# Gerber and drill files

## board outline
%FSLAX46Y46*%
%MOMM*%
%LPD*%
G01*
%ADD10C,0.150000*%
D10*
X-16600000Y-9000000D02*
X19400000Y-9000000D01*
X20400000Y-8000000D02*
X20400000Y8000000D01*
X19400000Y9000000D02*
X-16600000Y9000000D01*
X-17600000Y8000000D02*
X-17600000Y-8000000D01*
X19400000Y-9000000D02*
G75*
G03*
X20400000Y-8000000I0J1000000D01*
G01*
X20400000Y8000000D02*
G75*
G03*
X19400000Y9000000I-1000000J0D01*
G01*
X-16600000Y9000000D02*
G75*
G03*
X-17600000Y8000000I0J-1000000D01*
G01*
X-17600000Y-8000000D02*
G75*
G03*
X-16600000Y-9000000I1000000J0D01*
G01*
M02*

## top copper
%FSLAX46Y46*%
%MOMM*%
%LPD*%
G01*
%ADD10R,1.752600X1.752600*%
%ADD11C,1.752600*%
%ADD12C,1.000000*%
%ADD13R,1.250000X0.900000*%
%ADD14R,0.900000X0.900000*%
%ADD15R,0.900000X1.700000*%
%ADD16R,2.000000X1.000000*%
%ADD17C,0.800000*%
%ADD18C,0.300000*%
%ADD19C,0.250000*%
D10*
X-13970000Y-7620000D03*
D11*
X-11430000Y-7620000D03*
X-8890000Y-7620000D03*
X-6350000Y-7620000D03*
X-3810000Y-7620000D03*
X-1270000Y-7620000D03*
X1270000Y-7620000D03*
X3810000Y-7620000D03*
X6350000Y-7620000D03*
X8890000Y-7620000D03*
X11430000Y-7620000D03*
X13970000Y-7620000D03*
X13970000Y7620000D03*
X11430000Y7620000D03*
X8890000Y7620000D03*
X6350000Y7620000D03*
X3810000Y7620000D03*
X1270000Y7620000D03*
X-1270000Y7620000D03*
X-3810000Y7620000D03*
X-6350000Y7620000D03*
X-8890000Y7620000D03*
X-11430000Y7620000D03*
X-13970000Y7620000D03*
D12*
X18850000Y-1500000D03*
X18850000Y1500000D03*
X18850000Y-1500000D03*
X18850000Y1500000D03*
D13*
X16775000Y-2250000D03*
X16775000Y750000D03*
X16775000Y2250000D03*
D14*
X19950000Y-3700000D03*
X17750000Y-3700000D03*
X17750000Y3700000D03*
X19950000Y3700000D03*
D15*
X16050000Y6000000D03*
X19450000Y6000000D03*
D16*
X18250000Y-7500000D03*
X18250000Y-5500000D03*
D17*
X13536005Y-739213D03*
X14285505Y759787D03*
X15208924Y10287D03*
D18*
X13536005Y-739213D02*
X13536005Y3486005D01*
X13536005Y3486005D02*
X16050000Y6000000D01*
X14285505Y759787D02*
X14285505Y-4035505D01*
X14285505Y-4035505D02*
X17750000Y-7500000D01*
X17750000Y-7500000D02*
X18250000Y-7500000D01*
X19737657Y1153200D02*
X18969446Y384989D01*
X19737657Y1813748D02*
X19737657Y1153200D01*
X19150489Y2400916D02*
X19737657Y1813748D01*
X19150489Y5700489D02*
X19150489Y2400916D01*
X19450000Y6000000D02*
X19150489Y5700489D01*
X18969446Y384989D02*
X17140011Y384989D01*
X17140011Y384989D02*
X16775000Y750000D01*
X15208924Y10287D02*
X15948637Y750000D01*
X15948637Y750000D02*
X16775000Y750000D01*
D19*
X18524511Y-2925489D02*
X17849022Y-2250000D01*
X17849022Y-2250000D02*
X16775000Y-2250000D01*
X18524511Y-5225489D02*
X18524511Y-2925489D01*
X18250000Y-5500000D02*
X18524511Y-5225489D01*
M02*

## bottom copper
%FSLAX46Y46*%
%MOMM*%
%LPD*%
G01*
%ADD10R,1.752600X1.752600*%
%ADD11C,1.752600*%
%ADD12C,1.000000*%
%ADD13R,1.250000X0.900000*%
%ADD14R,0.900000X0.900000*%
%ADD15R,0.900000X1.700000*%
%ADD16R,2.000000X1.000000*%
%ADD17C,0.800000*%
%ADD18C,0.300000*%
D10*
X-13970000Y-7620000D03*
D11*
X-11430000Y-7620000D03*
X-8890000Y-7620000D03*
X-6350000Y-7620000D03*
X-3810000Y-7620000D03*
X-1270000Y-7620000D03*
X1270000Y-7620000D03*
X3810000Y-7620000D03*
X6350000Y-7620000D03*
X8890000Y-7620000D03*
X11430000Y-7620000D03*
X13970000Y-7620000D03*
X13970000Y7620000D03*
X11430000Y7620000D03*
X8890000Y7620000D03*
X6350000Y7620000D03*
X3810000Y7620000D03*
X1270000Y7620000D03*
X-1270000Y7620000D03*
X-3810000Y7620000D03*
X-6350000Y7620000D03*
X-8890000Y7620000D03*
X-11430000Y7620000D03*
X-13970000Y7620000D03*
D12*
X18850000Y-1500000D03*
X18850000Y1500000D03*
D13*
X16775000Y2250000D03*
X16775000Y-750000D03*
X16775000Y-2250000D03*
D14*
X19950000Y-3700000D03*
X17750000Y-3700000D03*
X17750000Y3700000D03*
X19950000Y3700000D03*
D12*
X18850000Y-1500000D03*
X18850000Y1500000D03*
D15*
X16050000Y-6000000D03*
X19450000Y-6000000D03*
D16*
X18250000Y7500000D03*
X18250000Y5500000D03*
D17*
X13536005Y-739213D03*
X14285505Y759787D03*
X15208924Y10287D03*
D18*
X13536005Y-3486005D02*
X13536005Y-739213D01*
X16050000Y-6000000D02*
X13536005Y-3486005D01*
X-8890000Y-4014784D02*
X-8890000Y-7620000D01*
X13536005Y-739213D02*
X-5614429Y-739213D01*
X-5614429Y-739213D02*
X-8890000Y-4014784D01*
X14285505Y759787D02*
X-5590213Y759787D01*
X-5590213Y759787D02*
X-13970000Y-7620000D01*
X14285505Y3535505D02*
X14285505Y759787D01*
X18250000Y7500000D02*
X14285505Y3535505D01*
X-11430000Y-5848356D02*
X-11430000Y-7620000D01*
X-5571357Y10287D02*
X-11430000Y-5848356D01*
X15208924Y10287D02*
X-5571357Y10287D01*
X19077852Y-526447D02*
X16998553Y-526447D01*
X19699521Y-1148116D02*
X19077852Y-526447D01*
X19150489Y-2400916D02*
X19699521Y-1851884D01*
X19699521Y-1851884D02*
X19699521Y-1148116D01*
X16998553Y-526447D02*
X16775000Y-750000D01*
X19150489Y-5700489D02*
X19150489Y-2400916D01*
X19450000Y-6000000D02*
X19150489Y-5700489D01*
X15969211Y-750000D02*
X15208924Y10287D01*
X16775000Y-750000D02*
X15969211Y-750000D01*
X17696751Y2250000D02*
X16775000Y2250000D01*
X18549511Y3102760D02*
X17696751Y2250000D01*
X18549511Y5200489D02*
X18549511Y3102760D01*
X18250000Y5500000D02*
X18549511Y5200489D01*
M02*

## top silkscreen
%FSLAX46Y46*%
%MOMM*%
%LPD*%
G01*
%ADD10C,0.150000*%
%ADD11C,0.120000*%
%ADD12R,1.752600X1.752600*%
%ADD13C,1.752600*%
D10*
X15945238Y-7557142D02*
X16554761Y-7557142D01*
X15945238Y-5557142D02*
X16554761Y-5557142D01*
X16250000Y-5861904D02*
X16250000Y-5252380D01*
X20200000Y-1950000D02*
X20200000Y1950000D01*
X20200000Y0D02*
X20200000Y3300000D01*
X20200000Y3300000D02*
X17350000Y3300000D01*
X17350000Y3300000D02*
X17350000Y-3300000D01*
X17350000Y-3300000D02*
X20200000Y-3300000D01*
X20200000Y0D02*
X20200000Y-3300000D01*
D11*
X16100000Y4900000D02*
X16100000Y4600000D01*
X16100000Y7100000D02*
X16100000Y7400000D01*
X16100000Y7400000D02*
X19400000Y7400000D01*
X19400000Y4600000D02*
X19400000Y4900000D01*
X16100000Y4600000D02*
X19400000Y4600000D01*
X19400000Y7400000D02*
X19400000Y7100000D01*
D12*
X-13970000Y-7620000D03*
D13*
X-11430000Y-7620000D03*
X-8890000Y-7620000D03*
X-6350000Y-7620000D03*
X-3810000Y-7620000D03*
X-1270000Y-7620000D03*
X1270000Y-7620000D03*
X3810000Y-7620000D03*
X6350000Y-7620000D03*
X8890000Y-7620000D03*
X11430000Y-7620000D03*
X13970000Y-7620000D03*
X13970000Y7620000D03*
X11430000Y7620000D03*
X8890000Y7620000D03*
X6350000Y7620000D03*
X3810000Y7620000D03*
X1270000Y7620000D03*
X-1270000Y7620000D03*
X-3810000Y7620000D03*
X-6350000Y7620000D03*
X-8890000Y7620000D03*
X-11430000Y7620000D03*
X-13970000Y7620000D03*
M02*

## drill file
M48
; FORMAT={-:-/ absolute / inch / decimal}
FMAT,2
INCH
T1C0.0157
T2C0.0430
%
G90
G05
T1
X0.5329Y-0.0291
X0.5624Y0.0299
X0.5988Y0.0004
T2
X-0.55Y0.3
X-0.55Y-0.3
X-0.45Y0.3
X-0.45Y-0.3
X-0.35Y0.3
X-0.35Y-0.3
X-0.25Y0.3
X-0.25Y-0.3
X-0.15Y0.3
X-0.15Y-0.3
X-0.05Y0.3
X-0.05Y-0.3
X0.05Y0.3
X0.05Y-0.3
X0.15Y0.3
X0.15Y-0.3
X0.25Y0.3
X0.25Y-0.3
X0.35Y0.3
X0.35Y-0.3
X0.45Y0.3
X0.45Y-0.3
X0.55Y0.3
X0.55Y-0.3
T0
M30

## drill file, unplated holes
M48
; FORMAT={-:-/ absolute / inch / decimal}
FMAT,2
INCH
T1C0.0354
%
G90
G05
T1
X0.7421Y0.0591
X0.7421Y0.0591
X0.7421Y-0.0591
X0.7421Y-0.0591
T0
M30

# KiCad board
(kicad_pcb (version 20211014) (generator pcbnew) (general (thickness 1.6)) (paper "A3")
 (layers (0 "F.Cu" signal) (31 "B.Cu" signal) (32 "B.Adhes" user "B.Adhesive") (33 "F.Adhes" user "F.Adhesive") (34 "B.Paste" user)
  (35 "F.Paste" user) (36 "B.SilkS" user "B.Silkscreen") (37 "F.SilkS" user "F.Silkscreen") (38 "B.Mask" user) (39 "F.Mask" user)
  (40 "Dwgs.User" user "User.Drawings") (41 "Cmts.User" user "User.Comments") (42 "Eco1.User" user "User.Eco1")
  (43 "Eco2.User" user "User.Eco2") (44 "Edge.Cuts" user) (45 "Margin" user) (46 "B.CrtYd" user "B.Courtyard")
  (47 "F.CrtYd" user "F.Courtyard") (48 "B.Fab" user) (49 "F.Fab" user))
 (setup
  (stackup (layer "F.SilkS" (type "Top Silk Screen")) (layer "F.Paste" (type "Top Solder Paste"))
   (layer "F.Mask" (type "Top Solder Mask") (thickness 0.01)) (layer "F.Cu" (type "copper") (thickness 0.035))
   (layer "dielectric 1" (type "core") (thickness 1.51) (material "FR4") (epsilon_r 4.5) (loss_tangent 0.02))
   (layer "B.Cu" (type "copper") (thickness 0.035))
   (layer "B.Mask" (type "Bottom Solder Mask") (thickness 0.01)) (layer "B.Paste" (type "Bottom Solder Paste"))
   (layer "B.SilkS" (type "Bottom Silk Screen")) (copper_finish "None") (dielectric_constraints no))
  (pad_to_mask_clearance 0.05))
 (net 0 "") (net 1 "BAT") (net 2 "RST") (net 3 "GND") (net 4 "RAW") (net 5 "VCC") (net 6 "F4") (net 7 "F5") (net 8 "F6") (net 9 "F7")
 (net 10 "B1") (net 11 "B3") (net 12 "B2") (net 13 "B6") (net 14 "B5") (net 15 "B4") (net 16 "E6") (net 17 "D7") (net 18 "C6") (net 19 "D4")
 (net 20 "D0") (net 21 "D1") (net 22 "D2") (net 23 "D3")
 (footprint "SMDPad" (layer "F.Cu") (at 18.25 -5.5)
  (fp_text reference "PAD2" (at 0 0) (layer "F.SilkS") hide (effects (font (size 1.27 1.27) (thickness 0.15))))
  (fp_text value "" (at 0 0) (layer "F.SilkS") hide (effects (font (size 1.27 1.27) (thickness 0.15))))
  (pad "1" smd rect locked (at 0 0) (size 2 1) (layers "B.Cu" "B.Paste" "B.Mask") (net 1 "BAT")))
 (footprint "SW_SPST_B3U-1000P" (layer "F.Cu") (at 17.75 -6)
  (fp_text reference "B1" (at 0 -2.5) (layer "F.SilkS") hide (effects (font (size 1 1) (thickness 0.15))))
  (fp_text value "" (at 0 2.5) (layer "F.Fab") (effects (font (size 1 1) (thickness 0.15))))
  (fp_line (start 1.65 -1.4) (end 1.65 -1.1) (layer "F.SilkS") (width 0.12))
  (fp_line (start -1.65 1.1) (end -1.65 1.4) (layer "F.SilkS") (width 0.12))
  (fp_line (start -1.65 1.4) (end 1.65 1.4) (layer "F.SilkS") (width 0.12))
  (fp_line (start 1.65 1.4) (end 1.65 1.1) (layer "F.SilkS") (width 0.12))
  (fp_line (start -1.65 -1.4) (end 1.65 -1.4) (layer "F.SilkS") (width 0.12))
  (fp_line (start -1.65 -1.1) (end -1.65 -1.4) (layer "F.SilkS") (width 0.12))
  (pad "1" smd rect locked (at -1.7 0) (size 0.9 1.7) (layers "F.Cu" "F.Paste" "F.Mask") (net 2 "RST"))
  (pad "2" smd rect locked (at 1.7 0) (size 0.9 1.7) (layers "F.Cu" "F.Paste" "F.Mask") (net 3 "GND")))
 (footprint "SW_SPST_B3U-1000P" (layer "F.Cu") (at 17.75 6)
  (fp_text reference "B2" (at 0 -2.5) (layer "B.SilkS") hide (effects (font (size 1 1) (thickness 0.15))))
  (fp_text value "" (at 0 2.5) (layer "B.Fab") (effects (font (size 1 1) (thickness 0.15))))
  (pad "1" smd rect locked (at -1.7 0) (size 0.9 1.7) (layers "B.Cu" "B.Paste" "B.Mask") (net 2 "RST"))
  (pad "2" smd rect locked (at 1.7 0) (size 0.9 1.7) (layers "B.Cu" "B.Paste" "B.Mask") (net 3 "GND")))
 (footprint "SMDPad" (layer "F.Cu") (at 18.25 5.5)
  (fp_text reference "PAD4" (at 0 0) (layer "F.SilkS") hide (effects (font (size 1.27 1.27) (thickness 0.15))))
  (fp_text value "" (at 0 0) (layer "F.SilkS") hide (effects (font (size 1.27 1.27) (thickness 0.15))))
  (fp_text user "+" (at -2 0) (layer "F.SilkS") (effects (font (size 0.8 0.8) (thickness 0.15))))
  (pad "1" smd rect locked (at 0 0) (size 2 1) (layers "F.Cu" "F.Paste" "F.Mask") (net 1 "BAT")))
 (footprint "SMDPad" (layer "F.Cu") (at 18.25 -7.5)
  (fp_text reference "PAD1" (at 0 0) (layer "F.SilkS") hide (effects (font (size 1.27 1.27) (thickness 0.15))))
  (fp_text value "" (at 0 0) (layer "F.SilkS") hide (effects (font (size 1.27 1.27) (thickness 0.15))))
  (pad "1" smd rect locked (at 0 0) (size 2 1) (layers "B.Cu" "B.Paste" "B.Mask") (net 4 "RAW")))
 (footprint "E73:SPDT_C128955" (layer "F.Cu") (at 18.85 0 -90)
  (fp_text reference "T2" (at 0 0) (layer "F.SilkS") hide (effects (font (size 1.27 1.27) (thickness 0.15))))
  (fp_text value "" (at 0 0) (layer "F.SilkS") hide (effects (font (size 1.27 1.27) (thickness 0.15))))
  (fp_line (start 0 -1.35) (end -3.3 -1.35) (layer "F.SilkS") (width 0.15))
  (fp_line (start 3.3 1.5) (end 3.3 -1.35) (layer "F.SilkS") (width 0.15))
  (fp_line (start -3.3 -1.35) (end -3.3 1.5) (layer "F.SilkS") (width 0.15))
  (fp_line (start -3.3 1.5) (end 3.3 1.5) (layer "F.SilkS") (width 0.15))
  (fp_line (start 0 -1.35) (end 3.3 -1.35) (layer "F.SilkS") (width 0.15))
  (fp_line (start 1.95 -1.35) (end -1.95 -1.35) (layer "F.SilkS") (width 0.15))
  (pad "" np_thru_hole circle locked (at 1.5 0) (size 1 1) (drill 0.9) (layers *.Cu *.Mask))
  (pad "" smd rect locked (at 3.7 -1.1 270) (size 0.9 0.9) (layers "F.Cu" "F.Paste" "F.Mask"))
  (pad "" smd rect locked (at 3.7 1.1 270) (size 0.9 0.9) (layers "F.Cu" "F.Paste" "F.Mask"))
  (pad "" np_thru_hole circle locked (at -1.5 0) (size 1 1) (drill 0.9) (layers *.Cu *.Mask))
  (pad "" smd rect locked (at -3.7 1.1 270) (size 0.9 0.9) (layers "F.Cu" "F.Paste" "F.Mask"))
  (pad "" smd rect locked (at -3.7 -1.1 270) (size 0.9 0.9) (layers "F.Cu" "F.Paste" "F.Mask"))
  (pad "1" smd rect locked (at 2.25 2.075 270) (size 0.9 1.25) (layers "F.Cu" "F.Paste" "F.Mask") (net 1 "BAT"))
  (pad "2" smd rect locked (at -0.75 2.075 270) (size 0.9 1.25) (layers "F.Cu" "F.Paste" "F.Mask") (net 3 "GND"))
  (pad "3" smd rect locked (at -2.25 2.075 270) (size 0.9 1.25) (layers "F.Cu" "F.Paste" "F.Mask")))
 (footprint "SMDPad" (layer "F.Cu") (at 18.25 7.5)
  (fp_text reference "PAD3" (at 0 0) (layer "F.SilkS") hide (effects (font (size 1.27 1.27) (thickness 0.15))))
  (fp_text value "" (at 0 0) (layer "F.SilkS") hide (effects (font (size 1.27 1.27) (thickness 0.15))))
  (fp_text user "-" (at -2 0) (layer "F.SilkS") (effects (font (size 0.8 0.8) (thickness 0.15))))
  (pad "1" smd rect locked (at 0 0) (size 2 1) (layers "F.Cu" "F.Paste" "F.Mask") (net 4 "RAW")))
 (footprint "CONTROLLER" (layer "F.Cu") (at 0 0)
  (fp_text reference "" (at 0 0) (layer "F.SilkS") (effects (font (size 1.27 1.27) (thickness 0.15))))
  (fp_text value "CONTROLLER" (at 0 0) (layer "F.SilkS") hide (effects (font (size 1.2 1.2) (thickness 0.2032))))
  (pad "1" thru_hole rect locked (at -13.97 7.62) (size 1.7526 1.7526) (drill 1.0922) (layers *.Cu *.SilkS *.Mask) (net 4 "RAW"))
  (pad "2" thru_hole circle locked (at -11.43 7.62) (size 1.7526 1.7526) (drill 1.0922) (layers *.Cu *.SilkS *.Mask) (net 3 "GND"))
  (pad "3" thru_hole circle locked (at -8.89 7.62) (size 1.7526 1.7526) (drill 1.0922) (layers *.Cu *.SilkS *.Mask) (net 2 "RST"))
  (pad "4" thru_hole circle locked (at -6.35 7.62) (size 1.7526 1.7526) (drill 1.0922) (layers *.Cu *.SilkS *.Mask) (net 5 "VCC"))
  (pad "5" thru_hole circle locked (at -3.81 7.62) (size 1.7526 1.7526) (drill 1.0922) (layers *.Cu *.SilkS *.Mask) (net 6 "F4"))
  (pad "6" thru_hole circle locked (at -1.27 7.62) (size 1.7526 1.7526) (drill 1.0922) (layers *.Cu *.SilkS *.Mask) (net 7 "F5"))
  (pad "7" thru_hole circle locked (at 1.27 7.62) (size 1.7526 1.7526) (drill 1.0922) (layers *.Cu *.SilkS *.Mask) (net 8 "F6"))
  (pad "8" thru_hole circle locked (at 3.81 7.62) (size 1.7526 1.7526) (drill 1.0922) (layers *.Cu *.SilkS *.Mask) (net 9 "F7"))
  (pad "9" thru_hole circle locked (at 6.35 7.62) (size 1.7526 1.7526) (drill 1.0922) (layers *.Cu *.SilkS *.Mask) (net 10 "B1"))
  (pad "10" thru_hole circle locked (at 8.89 7.62) (size 1.7526 1.7526) (drill 1.0922) (layers *.Cu *.SilkS *.Mask) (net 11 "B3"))
  (pad "11" thru_hole circle locked (at 11.43 7.62) (size 1.7526 1.7526) (drill 1.0922) (layers *.Cu *.SilkS *.Mask) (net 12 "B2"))
  (pad "12" thru_hole circle locked (at 13.97 7.62) (size 1.7526 1.7526) (drill 1.0922) (layers *.Cu *.SilkS *.Mask) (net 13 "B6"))
  (pad "13" thru_hole circle locked (at 13.97 -7.62) (size 1.7526 1.7526) (drill 1.0922) (layers *.Cu *.SilkS *.Mask) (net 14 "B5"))
  (pad "14" thru_hole circle locked (at 11.43 -7.62) (size 1.7526 1.7526) (drill 1.0922) (layers *.Cu *.SilkS *.Mask) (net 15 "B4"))
  (pad "15" thru_hole circle locked (at 8.89 -7.62) (size 1.7526 1.7526) (drill 1.0922) (layers *.Cu *.SilkS *.Mask) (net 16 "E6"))
  (pad "16" thru_hole circle locked (at 6.35 -7.62) (size 1.7526 1.7526) (drill 1.0922) (layers *.Cu *.SilkS *.Mask) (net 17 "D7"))
  (pad "17" thru_hole circle locked (at 3.81 -7.62) (size 1.7526 1.7526) (drill 1.0922) (layers *.Cu *.SilkS *.Mask) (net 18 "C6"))
  (pad "18" thru_hole circle locked (at 1.27 -7.62) (size 1.7526 1.7526) (drill 1.0922) (layers *.Cu *.SilkS *.Mask) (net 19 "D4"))
  (pad "19" thru_hole circle locked (at -1.27 -7.62) (size 1.7526 1.7526) (drill 1.0922) (layers *.Cu *.SilkS *.Mask) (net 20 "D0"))
  (pad "20" thru_hole circle locked (at -3.81 -7.62) (size 1.7526 1.7526) (drill 1.0922) (layers *.Cu *.SilkS *.Mask) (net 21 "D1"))
  (pad "21" thru_hole circle locked (at -6.35 -7.62) (size 1.7526 1.7526) (drill 1.0922) (layers *.Cu *.SilkS *.Mask) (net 3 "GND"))
  (pad "22" thru_hole circle locked (at -8.89 -7.62) (size 1.7526 1.7526) (drill 1.0922) (layers *.Cu *.SilkS *.Mask) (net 3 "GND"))
  (pad "23" thru_hole circle locked (at -11.43 -7.62) (size 1.7526 1.7526) (drill 1.0922) (layers *.Cu *.SilkS *.Mask) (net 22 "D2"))
  (pad "24" thru_hole circle locked (at -13.97 -7.62) (size 1.7526 1.7526) (drill 1.0922) (layers *.Cu *.SilkS *.Mask) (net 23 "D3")))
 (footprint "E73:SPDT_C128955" (layer "B.Cu") (at 18.85 0 -90)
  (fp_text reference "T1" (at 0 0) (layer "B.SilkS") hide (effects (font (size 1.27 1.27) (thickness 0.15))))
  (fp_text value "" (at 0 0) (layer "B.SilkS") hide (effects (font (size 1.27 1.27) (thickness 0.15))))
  (pad "" smd rect locked (at 3.7 -1.1 270) (size 0.9 0.9) (layers "B.Cu" "B.Paste" "B.Mask"))
  (pad "" smd rect locked (at -3.7 -1.1 270) (size 0.9 0.9) (layers "B.Cu" "B.Paste" "B.Mask"))
  (pad "" np_thru_hole circle locked (at 1.5 0) (size 1 1) (drill 0.9) (layers *.Cu *.Mask))
  (pad "" np_thru_hole circle locked (at -1.5 0) (size 1 1) (drill 0.9) (layers *.Cu *.Mask))
  (pad "" smd rect locked (at 3.7 1.1 270) (size 0.9 0.9) (layers "B.Cu" "B.Paste" "B.Mask"))
  (pad "" smd rect locked (at -3.7 1.1 270) (size 0.9 0.9) (layers "B.Cu" "B.Paste" "B.Mask"))
  (pad "1" smd rect locked (at -2.25 2.075 270) (size 0.9 1.25) (layers "B.Cu" "B.Paste" "B.Mask") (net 1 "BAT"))
  (pad "2" smd rect locked (at 0.75 2.075 270) (size 0.9 1.25) (layers "B.Cu" "B.Paste" "B.Mask") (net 3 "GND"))
  (pad "3" smd rect locked (at 2.25 2.075 270) (size 0.9 1.25) (layers "B.Cu" "B.Paste" "B.Mask")))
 (gr_line (start -17.6 -8) (end -17.6 8) (layer "Edge.Cuts") (width 0.15))
 (gr_arc (start -16.6 9) (mid -17.307107 8.707107) (end -17.6 8) (layer "Edge.Cuts") (width 0.15))
 (gr_arc (start 20.4 8) (mid 20.107107 8.707107) (end 19.4 9) (layer "Edge.Cuts") (width 0.15))
 (gr_line (start 19.4 -9) (end -16.6 -9) (layer "Edge.Cuts") (width 0.15))
 (gr_line (start 20.4 8) (end 20.4 -8) (layer "Edge.Cuts") (width 0.15))
 (gr_line (start -16.6 9) (end 19.4 9) (layer "Edge.Cuts") (width 0.15))
 (gr_arc (start -17.6 -8) (mid -17.307107 -8.707107) (end -16.6 -9) (layer "Edge.Cuts") (width 0.15))
 (gr_arc (start 19.4 -9) (mid 20.107107 -8.707107) (end 20.4 -8) (layer "Edge.Cuts") (width 0.15))
 (segment (start 14.285505 -0.759787) (end 14.285505 4.035505) (width 0.3) (layer "F.Cu") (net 4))
 (segment (start 17.75 7.5) (end 18.25 7.5) (width 0.3) (layer "F.Cu") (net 4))
 (segment (start 14.285505 4.035505) (end 17.75 7.5) (width 0.3) (layer "F.Cu") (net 4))
 (via (at 14.285505 -0.759787) (size 0.8) (drill 0.4) (layers "F.Cu" "B.Cu") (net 4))
 (segment (start -5.590213 -0.759787) (end -13.97 7.62) (width 0.3) (layer "B.Cu") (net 4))
 (segment (start 14.285505 -3.535505) (end 14.285505 -0.759787) (width 0.3) (layer "B.Cu") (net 4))
 (segment (start 14.285505 -0.759787) (end -5.590213 -0.759787) (width 0.3) (layer "B.Cu") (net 4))
 (segment (start 18.25 -7.5) (end 14.285505 -3.535505) (width 0.3) (layer "B.Cu") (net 4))
 (segment (start 19.45 -6) (end 19.150489 -5.700489) (width 0.3) (layer "F.Cu") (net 3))
 (segment (start 18.969446 -0.384989) (end 17.140011 -0.384989) (width 0.3) (layer "F.Cu") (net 3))
 (segment (start 19.737657 -1.813748) (end 19.737657 -1.1532) (width 0.3) (layer "F.Cu") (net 3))
 (segment (start 19.150489 -5.700489) (end 19.150489 -2.400916) (width 0.3) (layer "F.Cu") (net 3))
 (segment (start 15.208924 -0.010287) (end 15.948637 -0.75) (width 0.3) (layer "F.Cu") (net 3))
 (segment (start 15.948637 -0.75) (end 16.775 -0.75) (width 0.3) (layer "F.Cu") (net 3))
 (segment (start 17.140011 -0.384989) (end 16.775 -0.75) (width 0.3) (layer "F.Cu") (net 3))
 (segment (start 19.150489 -2.400916) (end 19.737657 -1.813748) (width 0.3) (layer "F.Cu") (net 3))
 (segment (start 19.737657 -1.1532) (end 18.969446 -0.384989) (width 0.3) (layer "F.Cu") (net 3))
 (via (at 15.208924 -0.010287) (size 0.8) (drill 0.4) (layers "F.Cu" "B.Cu") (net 3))
 (segment (start 16.775 0.75) (end 15.969211 0.75) (width 0.3) (layer "B.Cu") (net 3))
 (segment (start 19.45 6) (end 19.150489 5.700489) (width 0.3) (layer "B.Cu") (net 3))
 (segment (start 19.699521 1.851884) (end 19.699521 1.148116) (width 0.3) (layer "B.Cu") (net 3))
 (segment (start -11.43 5.848356) (end -11.43 7.62) (width 0.3) (layer "B.Cu") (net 3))
 (segment (start 19.150489 2.400916) (end 19.699521 1.851884) (width 0.3) (layer "B.Cu") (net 3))
 (segment (start 19.699521 1.148116) (end 19.077852 0.526447) (width 0.3) (layer "B.Cu") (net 3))
 (segment (start -5.571357 -0.010287) (end -11.43 5.848356) (width 0.3) (layer "B.Cu") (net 3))
 (segment (start 19.077852 0.526447) (end 16.998553 0.526447) (width 0.3) (layer "B.Cu") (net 3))
 (segment (start 15.208924 -0.010287) (end -5.571357 -0.010287) (width 0.3) (layer "B.Cu") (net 3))
 (segment (start 16.998553 0.526447) (end 16.775 0.75) (width 0.3) (layer "B.Cu") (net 3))
 (segment (start 15.969211 0.75) (end 15.208924 -0.010287) (width 0.3) (layer "B.Cu") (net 3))
 (segment (start 19.150489 5.700489) (end 19.150489 2.400916) (width 0.3) (layer "B.Cu") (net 3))
 (segment (start 13.536005 0.739213) (end 13.536005 -3.486005) (width 0.3) (layer "F.Cu") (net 2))
 (segment (start 13.536005 -3.486005) (end 16.05 -6) (width 0.3) (layer "F.Cu") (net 2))
 (via (at 13.536005 0.739213) (size 0.8) (drill 0.4) (layers "F.Cu" "B.Cu") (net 2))
 (segment (start -5.614429 0.739213) (end -8.89 4.014784) (width 0.3) (layer "B.Cu") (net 2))
 (segment (start 16.05 6) (end 13.536005 3.486005) (width 0.3) (layer "B.Cu") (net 2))
 (segment (start 13.536005 3.486005) (end 13.536005 0.739213) (width 0.3) (layer "B.Cu") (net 2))
 (segment (start -8.89 4.014784) (end -8.89 7.62) (width 0.3) (layer "B.Cu") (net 2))
 (segment (start 13.536005 0.739213) (end -5.614429 0.739213) (width 0.3) (layer "B.Cu") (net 2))
 (segment (start 18.524511 2.925489) (end 17.849022 2.25) (width 0.25) (layer "F.Cu") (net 1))
 (segment (start 17.849022 2.25) (end 16.775 2.25) (width 0.25) (layer "F.Cu") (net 1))
 (segment (start 18.524511 5.225489) (end 18.524511 2.925489) (width 0.25) (layer "F.Cu") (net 1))
 (segment (start 18.25 5.5) (end 18.524511 5.225489) (width 0.25) (layer "F.Cu") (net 1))
 (segment (start 18.549511 -5.200489) (end 18.549511 -3.10276) (width 0.3) (layer "B.Cu") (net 1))
 (segment (start 17.696751 -2.25) (end 16.775 -2.25) (width 0.3) (layer "B.Cu") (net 1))
 (segment (start 18.549511 -3.10276) (end 17.696751 -2.25) (width 0.3) (layer "B.Cu") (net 1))
 (segment (start 18.25 -5.5) (end 18.549511 -5.200489) (width 0.3) (layer "B.Cu") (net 1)))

